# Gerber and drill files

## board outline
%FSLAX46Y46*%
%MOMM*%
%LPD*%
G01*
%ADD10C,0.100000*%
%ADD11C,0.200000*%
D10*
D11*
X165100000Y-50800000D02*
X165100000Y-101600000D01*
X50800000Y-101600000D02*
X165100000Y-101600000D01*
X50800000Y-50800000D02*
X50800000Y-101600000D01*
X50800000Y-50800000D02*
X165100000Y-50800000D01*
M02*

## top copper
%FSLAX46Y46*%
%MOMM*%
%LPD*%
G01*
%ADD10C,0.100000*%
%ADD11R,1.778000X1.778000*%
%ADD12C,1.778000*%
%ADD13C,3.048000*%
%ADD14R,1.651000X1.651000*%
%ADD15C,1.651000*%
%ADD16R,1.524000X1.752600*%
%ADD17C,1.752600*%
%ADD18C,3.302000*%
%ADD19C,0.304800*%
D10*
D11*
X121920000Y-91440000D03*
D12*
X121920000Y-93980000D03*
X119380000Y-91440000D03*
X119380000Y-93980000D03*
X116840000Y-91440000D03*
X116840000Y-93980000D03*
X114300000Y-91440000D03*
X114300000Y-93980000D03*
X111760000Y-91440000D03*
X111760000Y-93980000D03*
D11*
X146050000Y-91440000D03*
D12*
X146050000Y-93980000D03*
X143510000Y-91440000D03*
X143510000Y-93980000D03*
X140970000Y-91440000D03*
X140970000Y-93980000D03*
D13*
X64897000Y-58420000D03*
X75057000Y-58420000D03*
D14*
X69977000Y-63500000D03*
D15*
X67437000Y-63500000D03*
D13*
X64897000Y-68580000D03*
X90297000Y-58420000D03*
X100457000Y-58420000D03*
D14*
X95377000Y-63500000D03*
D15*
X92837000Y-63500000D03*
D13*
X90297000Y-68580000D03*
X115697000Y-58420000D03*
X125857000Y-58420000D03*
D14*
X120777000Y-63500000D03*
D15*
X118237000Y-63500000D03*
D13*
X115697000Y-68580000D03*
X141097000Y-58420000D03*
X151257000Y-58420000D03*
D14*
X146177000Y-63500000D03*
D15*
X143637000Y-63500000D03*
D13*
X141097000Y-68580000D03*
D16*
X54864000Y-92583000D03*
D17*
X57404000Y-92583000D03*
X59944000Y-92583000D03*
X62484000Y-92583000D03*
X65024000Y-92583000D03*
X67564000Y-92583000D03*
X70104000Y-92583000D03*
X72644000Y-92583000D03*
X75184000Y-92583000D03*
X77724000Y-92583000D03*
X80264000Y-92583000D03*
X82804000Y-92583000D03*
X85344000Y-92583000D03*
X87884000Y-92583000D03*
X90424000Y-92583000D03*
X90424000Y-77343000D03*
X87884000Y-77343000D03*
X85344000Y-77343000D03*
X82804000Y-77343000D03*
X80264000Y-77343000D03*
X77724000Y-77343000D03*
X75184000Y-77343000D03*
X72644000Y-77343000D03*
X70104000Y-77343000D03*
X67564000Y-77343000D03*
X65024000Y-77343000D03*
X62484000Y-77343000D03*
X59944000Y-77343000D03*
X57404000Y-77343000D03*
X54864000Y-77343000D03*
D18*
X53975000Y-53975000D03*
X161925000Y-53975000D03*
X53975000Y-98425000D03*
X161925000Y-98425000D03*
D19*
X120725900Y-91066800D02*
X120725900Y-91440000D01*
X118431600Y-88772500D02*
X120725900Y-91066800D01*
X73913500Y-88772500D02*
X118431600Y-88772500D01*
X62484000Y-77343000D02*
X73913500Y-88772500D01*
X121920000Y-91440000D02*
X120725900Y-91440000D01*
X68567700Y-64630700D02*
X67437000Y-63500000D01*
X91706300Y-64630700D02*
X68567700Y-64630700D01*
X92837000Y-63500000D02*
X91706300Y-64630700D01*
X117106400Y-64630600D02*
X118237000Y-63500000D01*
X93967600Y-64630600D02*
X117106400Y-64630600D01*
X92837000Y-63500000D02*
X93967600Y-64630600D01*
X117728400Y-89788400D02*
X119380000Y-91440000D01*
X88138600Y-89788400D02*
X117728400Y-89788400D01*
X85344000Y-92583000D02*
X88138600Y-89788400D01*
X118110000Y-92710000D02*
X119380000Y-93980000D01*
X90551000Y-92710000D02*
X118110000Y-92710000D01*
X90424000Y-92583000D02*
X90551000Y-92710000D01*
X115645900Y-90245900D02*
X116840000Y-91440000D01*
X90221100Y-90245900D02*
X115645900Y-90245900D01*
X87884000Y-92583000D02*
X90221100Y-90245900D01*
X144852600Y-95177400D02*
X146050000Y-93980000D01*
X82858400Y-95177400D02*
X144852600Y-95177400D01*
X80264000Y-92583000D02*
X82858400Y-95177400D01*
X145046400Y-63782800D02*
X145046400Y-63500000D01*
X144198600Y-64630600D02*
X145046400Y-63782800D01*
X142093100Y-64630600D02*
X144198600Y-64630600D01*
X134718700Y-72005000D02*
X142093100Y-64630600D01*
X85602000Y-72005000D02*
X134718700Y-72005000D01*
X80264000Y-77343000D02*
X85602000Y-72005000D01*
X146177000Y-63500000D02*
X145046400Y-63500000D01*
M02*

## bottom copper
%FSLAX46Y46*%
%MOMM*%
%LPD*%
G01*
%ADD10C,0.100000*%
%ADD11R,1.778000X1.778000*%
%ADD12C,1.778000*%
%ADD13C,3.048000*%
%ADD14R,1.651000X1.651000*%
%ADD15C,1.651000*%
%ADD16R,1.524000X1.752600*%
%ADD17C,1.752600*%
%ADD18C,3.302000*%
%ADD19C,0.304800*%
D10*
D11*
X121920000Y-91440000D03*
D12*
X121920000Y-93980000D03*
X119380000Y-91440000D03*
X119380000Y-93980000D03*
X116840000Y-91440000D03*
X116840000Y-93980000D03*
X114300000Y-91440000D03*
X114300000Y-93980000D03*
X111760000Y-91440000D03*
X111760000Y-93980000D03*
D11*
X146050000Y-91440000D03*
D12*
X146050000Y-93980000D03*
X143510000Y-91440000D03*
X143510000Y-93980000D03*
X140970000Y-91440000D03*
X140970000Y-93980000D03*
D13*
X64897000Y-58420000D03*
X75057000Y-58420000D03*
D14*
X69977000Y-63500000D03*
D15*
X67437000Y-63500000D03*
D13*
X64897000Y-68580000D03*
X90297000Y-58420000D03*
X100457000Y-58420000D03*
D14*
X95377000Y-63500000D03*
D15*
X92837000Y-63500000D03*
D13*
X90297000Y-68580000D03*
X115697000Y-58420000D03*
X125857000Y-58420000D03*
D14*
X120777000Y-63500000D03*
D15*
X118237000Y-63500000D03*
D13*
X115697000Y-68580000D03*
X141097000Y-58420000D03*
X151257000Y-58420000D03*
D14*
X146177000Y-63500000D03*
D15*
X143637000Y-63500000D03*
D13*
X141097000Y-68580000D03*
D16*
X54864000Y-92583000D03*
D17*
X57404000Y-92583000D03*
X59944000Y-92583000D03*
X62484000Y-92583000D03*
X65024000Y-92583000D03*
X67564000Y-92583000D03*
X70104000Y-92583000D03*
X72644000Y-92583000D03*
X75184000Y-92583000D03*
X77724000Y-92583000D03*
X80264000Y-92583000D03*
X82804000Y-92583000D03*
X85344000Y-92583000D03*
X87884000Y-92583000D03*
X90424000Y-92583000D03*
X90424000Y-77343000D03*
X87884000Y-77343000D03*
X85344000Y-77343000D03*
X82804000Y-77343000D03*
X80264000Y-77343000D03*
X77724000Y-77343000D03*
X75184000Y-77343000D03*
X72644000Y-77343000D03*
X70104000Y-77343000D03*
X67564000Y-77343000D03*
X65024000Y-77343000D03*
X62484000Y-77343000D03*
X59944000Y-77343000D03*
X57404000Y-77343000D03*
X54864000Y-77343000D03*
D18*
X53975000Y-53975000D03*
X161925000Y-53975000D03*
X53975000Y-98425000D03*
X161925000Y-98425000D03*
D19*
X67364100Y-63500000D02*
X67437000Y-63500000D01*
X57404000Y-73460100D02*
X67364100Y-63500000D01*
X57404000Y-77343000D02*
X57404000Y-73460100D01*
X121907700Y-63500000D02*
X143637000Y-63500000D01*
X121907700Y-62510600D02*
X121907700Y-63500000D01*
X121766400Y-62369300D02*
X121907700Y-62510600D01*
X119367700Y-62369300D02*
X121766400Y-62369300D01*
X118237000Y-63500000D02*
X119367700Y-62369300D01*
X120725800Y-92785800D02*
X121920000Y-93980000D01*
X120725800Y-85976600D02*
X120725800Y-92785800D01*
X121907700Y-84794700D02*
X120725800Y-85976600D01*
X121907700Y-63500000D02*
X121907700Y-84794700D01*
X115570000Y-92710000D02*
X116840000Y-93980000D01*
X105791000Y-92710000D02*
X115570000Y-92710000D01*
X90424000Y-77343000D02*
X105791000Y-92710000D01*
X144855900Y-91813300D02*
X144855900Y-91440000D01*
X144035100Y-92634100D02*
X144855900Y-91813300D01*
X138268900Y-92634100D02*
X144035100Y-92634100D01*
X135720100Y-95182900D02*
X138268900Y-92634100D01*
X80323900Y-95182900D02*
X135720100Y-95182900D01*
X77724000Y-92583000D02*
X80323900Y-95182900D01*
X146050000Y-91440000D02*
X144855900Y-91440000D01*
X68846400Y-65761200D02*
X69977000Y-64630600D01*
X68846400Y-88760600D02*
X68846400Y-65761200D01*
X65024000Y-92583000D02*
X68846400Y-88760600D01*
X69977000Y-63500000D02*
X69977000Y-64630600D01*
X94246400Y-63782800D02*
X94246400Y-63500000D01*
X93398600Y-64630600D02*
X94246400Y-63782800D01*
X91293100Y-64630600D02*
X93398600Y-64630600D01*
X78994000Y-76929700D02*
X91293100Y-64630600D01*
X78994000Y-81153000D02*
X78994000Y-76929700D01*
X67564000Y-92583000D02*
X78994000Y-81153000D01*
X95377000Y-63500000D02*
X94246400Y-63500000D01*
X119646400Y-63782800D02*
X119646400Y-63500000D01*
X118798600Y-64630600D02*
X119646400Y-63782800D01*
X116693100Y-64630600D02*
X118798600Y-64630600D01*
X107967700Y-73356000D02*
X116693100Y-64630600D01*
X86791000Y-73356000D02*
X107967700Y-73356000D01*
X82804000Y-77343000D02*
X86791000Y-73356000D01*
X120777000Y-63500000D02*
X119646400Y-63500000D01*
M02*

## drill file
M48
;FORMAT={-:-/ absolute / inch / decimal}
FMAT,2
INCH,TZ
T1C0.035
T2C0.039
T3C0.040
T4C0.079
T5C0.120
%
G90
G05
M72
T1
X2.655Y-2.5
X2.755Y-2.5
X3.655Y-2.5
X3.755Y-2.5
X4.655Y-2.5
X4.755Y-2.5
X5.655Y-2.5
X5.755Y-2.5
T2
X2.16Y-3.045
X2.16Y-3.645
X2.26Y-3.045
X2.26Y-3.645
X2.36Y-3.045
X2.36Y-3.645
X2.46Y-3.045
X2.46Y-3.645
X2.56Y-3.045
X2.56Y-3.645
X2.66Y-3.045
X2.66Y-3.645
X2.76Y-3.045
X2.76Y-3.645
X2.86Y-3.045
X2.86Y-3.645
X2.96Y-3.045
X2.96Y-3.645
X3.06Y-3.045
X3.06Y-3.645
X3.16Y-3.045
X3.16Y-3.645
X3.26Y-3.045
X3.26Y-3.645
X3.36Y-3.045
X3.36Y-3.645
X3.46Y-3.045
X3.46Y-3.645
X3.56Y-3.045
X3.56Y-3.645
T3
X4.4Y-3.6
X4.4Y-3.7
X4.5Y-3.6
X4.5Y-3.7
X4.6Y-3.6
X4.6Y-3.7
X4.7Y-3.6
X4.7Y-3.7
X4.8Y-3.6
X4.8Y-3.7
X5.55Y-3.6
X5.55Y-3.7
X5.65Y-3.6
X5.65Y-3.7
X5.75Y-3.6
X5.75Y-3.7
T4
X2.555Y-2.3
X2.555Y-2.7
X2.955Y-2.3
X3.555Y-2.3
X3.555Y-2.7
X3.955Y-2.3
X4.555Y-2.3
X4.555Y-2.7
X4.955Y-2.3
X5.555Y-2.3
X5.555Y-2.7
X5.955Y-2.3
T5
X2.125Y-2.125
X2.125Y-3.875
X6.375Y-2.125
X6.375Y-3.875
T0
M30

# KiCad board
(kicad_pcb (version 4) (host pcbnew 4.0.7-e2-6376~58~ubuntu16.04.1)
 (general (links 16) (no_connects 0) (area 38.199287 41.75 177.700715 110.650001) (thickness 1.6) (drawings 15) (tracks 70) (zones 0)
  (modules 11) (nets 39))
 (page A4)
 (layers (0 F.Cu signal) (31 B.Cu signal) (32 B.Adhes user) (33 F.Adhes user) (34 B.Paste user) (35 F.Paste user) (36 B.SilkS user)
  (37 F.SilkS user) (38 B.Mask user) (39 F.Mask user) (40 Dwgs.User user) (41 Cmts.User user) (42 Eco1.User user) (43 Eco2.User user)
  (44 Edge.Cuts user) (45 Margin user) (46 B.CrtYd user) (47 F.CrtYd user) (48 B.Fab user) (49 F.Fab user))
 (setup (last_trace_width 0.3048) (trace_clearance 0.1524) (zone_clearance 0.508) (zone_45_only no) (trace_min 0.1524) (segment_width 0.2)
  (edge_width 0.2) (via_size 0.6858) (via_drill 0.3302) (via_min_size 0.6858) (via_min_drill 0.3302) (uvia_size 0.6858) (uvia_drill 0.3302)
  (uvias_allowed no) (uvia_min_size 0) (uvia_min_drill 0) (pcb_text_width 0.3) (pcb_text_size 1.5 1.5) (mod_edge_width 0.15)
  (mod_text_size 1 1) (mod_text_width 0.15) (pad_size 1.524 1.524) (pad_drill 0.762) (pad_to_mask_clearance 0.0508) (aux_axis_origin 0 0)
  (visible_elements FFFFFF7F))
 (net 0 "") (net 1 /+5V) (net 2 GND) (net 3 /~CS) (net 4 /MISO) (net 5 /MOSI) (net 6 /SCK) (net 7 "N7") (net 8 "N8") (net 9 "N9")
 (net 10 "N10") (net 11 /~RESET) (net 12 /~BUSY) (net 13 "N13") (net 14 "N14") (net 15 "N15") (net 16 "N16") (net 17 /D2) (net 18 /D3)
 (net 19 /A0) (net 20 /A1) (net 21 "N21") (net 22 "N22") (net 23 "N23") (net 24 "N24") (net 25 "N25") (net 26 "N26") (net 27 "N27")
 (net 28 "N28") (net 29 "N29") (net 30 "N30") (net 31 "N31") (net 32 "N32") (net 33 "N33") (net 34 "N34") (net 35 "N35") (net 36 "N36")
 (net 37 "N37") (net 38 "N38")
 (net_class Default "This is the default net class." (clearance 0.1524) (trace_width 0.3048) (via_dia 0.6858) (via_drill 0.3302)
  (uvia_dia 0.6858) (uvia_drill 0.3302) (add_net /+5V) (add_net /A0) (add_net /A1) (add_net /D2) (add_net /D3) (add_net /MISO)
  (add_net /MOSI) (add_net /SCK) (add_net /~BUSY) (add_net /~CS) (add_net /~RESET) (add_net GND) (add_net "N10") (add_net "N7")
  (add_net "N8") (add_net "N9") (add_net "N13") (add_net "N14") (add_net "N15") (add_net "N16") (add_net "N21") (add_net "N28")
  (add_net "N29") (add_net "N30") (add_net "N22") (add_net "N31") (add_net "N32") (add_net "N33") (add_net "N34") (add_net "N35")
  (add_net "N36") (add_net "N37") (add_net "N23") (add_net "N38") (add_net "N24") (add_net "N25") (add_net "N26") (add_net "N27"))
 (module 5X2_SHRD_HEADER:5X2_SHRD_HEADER (layer F.Cu) (at 116.84 92.71 180)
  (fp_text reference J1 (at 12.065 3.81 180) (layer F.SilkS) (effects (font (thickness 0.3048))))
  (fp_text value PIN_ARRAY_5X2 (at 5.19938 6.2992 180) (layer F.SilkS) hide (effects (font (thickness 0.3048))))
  (pad 1 thru_hole rect (at -5.08 1.27 180) (size 1.778 1.778) (drill 1.016) (layers *.Cu *.Mask F.SilkS) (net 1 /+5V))
  (pad 2 thru_hole circle (at -5.08 -1.27 180) (size 1.778 1.778) (drill 1.016) (layers *.Cu *.Mask F.SilkS) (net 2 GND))
  (pad 3 thru_hole circle (at -2.54 1.27 180) (size 1.778 1.778) (drill 1.016) (layers *.Cu *.Mask F.SilkS) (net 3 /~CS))
  (pad 4 thru_hole circle (at -2.54 -1.27 180) (size 1.778 1.778) (drill 1.016) (layers *.Cu *.Mask F.SilkS) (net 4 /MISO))
  (pad 5 thru_hole circle (at 0 1.27 180) (size 1.778 1.778) (drill 1.016) (layers *.Cu *.Mask F.SilkS) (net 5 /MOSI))
  (pad 6 thru_hole circle (at 0 -1.27 180) (size 1.778 1.778) (drill 1.016) (layers *.Cu *.Mask F.SilkS) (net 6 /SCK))
  (pad 7 thru_hole circle (at 2.54 1.27 180) (size 1.778 1.778) (drill 1.016) (layers *.Cu *.Mask F.SilkS) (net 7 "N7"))
  (pad 8 thru_hole circle (at 2.54 -1.27 180) (size 1.778 1.778) (drill 1.016) (layers *.Cu *.Mask F.SilkS) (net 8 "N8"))
  (pad 9 thru_hole circle (at 5.08 1.27 180) (size 1.778 1.778) (drill 1.016) (layers *.Cu *.Mask F.SilkS) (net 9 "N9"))
  (pad 10 thru_hole circle (at 5.08 -1.27 180) (size 1.778 1.778) (drill 1.016) (layers *.Cu *.Mask F.SilkS) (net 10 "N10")))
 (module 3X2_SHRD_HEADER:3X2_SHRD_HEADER (layer F.Cu) (at 143.51 92.71 180)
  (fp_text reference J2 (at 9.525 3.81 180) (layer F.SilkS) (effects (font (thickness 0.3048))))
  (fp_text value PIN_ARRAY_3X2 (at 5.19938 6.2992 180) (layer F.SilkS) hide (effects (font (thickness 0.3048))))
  (pad 1 thru_hole rect (at -2.54 1.27 180) (size 1.778 1.778) (drill 1.016) (layers *.Cu *.Mask F.SilkS) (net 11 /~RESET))
  (pad 2 thru_hole circle (at -2.54 -1.27 180) (size 1.778 1.778) (drill 1.016) (layers *.Cu *.Mask F.SilkS) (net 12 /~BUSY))
  (pad 3 thru_hole circle (at 0 1.27 180) (size 1.778 1.778) (drill 1.016) (layers *.Cu *.Mask F.SilkS) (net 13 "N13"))
  (pad 4 thru_hole circle (at 0 -1.27 180) (size 1.778 1.778) (drill 1.016) (layers *.Cu *.Mask F.SilkS) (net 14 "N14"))
  (pad 5 thru_hole circle (at 2.54 1.27 180) (size 1.778 1.778) (drill 1.016) (layers *.Cu *.Mask F.SilkS) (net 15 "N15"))
  (pad 6 thru_hole circle (at 2.54 -1.27 180) (size 1.778 1.778) (drill 1.016) (layers *.Cu *.Mask F.SilkS) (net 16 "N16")))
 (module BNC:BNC (layer F.Cu) (at 69.977 58.42)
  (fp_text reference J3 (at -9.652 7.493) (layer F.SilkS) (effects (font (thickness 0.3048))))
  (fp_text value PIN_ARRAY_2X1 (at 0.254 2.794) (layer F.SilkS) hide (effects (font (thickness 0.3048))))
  (pad "" thru_hole circle (at -5.08 0) (size 3.048 3.048) (drill 2.00914) (layers *.Cu *.Mask))
  (pad "" thru_hole circle (at 5.08 0) (size 3.048 3.048) (drill 2.00914) (layers *.Cu *.Mask))
  (pad 1 thru_hole rect (at 0 5.08) (size 1.651 1.651) (drill 0.889) (layers *.Cu *.Mask) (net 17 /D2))
  (pad 2 thru_hole circle (at -2.54 5.08) (size 1.651 1.651) (drill 0.889) (layers *.Cu *.Mask) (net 2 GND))
  (pad "" thru_hole circle (at -5.08 10.16) (size 3.048 3.048) (drill 2.00914) (layers *.Cu *.Mask)))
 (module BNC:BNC (layer F.Cu) (at 95.377 58.42)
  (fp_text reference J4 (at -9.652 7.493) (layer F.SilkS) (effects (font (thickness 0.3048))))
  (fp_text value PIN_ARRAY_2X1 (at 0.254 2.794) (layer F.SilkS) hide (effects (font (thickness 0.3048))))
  (pad "" thru_hole circle (at -5.08 0) (size 3.048 3.048) (drill 2.00914) (layers *.Cu *.Mask))
  (pad "" thru_hole circle (at 5.08 0) (size 3.048 3.048) (drill 2.00914) (layers *.Cu *.Mask))
  (pad 1 thru_hole rect (at 0 5.08) (size 1.651 1.651) (drill 0.889) (layers *.Cu *.Mask) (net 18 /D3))
  (pad 2 thru_hole circle (at -2.54 5.08) (size 1.651 1.651) (drill 0.889) (layers *.Cu *.Mask) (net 2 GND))
  (pad "" thru_hole circle (at -5.08 10.16) (size 3.048 3.048) (drill 2.00914) (layers *.Cu *.Mask)))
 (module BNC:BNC (layer F.Cu) (at 120.777 58.42)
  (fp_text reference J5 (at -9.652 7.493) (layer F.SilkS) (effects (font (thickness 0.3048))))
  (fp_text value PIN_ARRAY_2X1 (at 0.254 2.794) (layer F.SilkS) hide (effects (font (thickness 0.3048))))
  (pad "" thru_hole circle (at -5.08 0) (size 3.048 3.048) (drill 2.00914) (layers *.Cu *.Mask))
  (pad "" thru_hole circle (at 5.08 0) (size 3.048 3.048) (drill 2.00914) (layers *.Cu *.Mask))
  (pad 1 thru_hole rect (at 0 5.08) (size 1.651 1.651) (drill 0.889) (layers *.Cu *.Mask) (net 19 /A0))
  (pad 2 thru_hole circle (at -2.54 5.08) (size 1.651 1.651) (drill 0.889) (layers *.Cu *.Mask) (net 2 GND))
  (pad "" thru_hole circle (at -5.08 10.16) (size 3.048 3.048) (drill 2.00914) (layers *.Cu *.Mask)))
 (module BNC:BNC (layer F.Cu) (at 146.177 58.42)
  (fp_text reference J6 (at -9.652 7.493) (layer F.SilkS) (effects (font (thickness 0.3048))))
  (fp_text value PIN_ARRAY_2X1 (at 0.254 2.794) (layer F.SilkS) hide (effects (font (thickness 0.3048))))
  (pad "" thru_hole circle (at -5.08 0) (size 3.048 3.048) (drill 2.00914) (layers *.Cu *.Mask))
  (pad "" thru_hole circle (at 5.08 0) (size 3.048 3.048) (drill 2.00914) (layers *.Cu *.Mask))
  (pad 1 thru_hole rect (at 0 5.08) (size 1.651 1.651) (drill 0.889) (layers *.Cu *.Mask) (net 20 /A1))
  (pad 2 thru_hole circle (at -2.54 5.08) (size 1.651 1.651) (drill 0.889) (layers *.Cu *.Mask) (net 2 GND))
  (pad "" thru_hole circle (at -5.08 10.16) (size 3.048 3.048) (drill 2.00914) (layers *.Cu *.Mask)))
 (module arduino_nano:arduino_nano (layer F.Cu) (at 72.644 84.963 90)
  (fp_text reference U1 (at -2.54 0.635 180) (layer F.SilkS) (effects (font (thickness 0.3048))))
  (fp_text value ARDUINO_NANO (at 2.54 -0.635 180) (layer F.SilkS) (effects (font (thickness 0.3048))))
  (pad 1 thru_hole rect (at -7.62 -17.78 90) (size 1.7526 1.524) (drill 0.9906) (layers *.Cu *.Mask F.SilkS) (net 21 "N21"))
  (pad 2 thru_hole circle (at -7.62 -15.24 90) (size 1.7526 1.7526) (drill 0.9906) (layers *.Cu *.Mask F.SilkS) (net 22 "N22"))
  (pad 3 thru_hole circle (at -7.62 -12.7 90) (size 1.7526 1.7526) (drill 0.9906) (layers *.Cu *.Mask F.SilkS) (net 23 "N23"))
  (pad 4 thru_hole circle (at -7.62 -10.16 90) (size 1.7526 1.7526) (drill 0.9906) (layers *.Cu *.Mask F.SilkS) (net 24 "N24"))
  (pad 5 thru_hole circle (at -7.62 -7.62 90) (size 1.7526 1.7526) (drill 0.9906) (layers *.Cu *.Mask F.SilkS) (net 17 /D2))
  (pad 6 thru_hole circle (at -7.62 -5.08 90) (size 1.7526 1.7526) (drill 0.9906) (layers *.Cu *.Mask F.SilkS) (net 18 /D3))
  (pad 7 thru_hole circle (at -7.62 -2.54 90) (size 1.7526 1.7526) (drill 0.9906) (layers *.Cu *.Mask F.SilkS) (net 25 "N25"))
  (pad 8 thru_hole circle (at -7.62 0 90) (size 1.7526 1.7526) (drill 0.9906) (layers *.Cu *.Mask F.SilkS) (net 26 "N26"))
  (pad 9 thru_hole circle (at -7.62 2.54 90) (size 1.7526 1.7526) (drill 0.9906) (layers *.Cu *.Mask F.SilkS) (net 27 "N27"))
  (pad 10 thru_hole circle (at -7.62 5.08 90) (size 1.7526 1.7526) (drill 0.9906) (layers *.Cu *.Mask F.SilkS) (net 11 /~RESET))
  (pad 11 thru_hole circle (at -7.62 7.62 90) (size 1.7526 1.7526) (drill 0.9906) (layers *.Cu *.Mask F.SilkS) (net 12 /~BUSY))
  (pad 12 thru_hole circle (at -7.62 10.16 90) (size 1.7526 1.7526) (drill 0.9906) (layers *.Cu *.Mask F.SilkS) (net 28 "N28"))
  (pad 13 thru_hole circle (at -7.62 12.7 90) (size 1.7526 1.7526) (drill 0.9906) (layers *.Cu *.Mask F.SilkS) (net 3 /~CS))
  (pad 14 thru_hole circle (at -7.62 15.24 90) (size 1.7526 1.7526) (drill 0.9906) (layers *.Cu *.Mask F.SilkS) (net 5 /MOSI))
  (pad 15 thru_hole circle (at -7.62 17.78 90) (size 1.7526 1.7526) (drill 0.9906) (layers *.Cu *.Mask F.SilkS) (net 4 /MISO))
  (pad 16 thru_hole circle (at 7.62 17.78 90) (size 1.7526 1.7526) (drill 0.9906) (layers *.Cu *.Mask F.SilkS) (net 6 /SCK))
  (pad 17 thru_hole circle (at 7.62 15.24 90) (size 1.7526 1.7526) (drill 0.9906) (layers *.Cu *.Mask F.SilkS) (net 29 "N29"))
  (pad 18 thru_hole circle (at 7.62 12.7 90) (size 1.7526 1.7526) (drill 0.9906) (layers *.Cu *.Mask F.SilkS) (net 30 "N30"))
  (pad 19 thru_hole circle (at 7.62 10.16 90) (size 1.7526 1.7526) (drill 0.9906) (layers *.Cu *.Mask F.SilkS) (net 19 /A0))
  (pad 20 thru_hole circle (at 7.62 7.62 90) (size 1.7526 1.7526) (drill 0.9906) (layers *.Cu *.Mask F.SilkS) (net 20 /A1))
  (pad 21 thru_hole circle (at 7.62 5.08 90) (size 1.7526 1.7526) (drill 0.9906) (layers *.Cu *.Mask F.SilkS) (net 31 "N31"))
  (pad 22 thru_hole circle (at 7.62 2.54 90) (size 1.7526 1.7526) (drill 0.9906) (layers *.Cu *.Mask F.SilkS) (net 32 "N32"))
  (pad 23 thru_hole circle (at 7.62 0 90) (size 1.7526 1.7526) (drill 0.9906) (layers *.Cu *.Mask F.SilkS) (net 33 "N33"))
  (pad 24 thru_hole circle (at 7.62 -2.54 90) (size 1.7526 1.7526) (drill 0.9906) (layers *.Cu *.Mask F.SilkS) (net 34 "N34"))
  (pad 25 thru_hole circle (at 7.62 -5.08 90) (size 1.7526 1.7526) (drill 0.9906) (layers *.Cu *.Mask F.SilkS) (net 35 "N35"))
  (pad 26 thru_hole circle (at 7.62 -7.62 90) (size 1.7526 1.7526) (drill 0.9906) (layers *.Cu *.Mask F.SilkS) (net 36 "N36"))
  (pad 27 thru_hole circle (at 7.62 -10.16 90) (size 1.7526 1.7526) (drill 0.9906) (layers *.Cu *.Mask F.SilkS) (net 1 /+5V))
  (pad 28 thru_hole circle (at 7.62 -12.7 90) (size 1.7526 1.7526) (drill 0.9906) (layers *.Cu *.Mask F.SilkS) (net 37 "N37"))
  (pad 29 thru_hole circle (at 7.62 -15.24 90) (size 1.7526 1.7526) (drill 0.9906) (layers *.Cu *.Mask F.SilkS) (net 2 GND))
  (pad 30 thru_hole circle (at 7.62 -17.78 90) (size 1.7526 1.7526) (drill 0.9906) (layers *.Cu *.Mask F.SilkS) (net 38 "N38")))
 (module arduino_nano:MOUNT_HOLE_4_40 (layer F.Cu) (at 53.975 53.975)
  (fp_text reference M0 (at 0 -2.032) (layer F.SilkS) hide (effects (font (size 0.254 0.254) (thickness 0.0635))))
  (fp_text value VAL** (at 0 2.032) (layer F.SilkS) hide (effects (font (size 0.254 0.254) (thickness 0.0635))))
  (pad "" thru_hole circle (at 0 0) (size 3.302 3.302) (drill 3.048) (layers *.Cu *.SilkS *.Mask)))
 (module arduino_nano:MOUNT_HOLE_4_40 (layer F.Cu) (at 161.925 53.975)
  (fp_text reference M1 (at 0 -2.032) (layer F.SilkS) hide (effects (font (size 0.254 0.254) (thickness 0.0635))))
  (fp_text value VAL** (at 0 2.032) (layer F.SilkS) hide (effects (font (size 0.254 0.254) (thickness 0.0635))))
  (pad "" thru_hole circle (at 0 0) (size 3.302 3.302) (drill 3.048) (layers *.Cu *.SilkS *.Mask)))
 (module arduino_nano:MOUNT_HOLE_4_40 (layer F.Cu) (at 53.975 98.425)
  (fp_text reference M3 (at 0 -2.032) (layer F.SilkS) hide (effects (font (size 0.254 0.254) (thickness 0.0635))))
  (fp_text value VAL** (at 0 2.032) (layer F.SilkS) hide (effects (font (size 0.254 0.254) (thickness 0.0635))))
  (pad "" thru_hole circle (at 0 0) (size 3.302 3.302) (drill 3.048) (layers *.Cu *.SilkS *.Mask)))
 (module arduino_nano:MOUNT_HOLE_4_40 (layer F.Cu) (at 161.925 98.425)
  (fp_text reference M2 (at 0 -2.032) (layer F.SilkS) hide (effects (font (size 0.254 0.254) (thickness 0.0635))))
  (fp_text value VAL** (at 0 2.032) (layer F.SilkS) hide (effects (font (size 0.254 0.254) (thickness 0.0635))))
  (pad "" thru_hole circle (at 0 0) (size 3.302 3.302) (drill 3.048) (layers *.Cu *.SilkS *.Mask)))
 (gr_line (start 165.1 50.8) (end 165.1 101.6) (angle 90) (layer Edge.Cuts) (width 0.2))
 (gr_line (start 50.8 101.6) (end 165.1 101.6) (angle 90) (layer Edge.Cuts) (width 0.2))
 (gr_line (start 50.8 50.8) (end 50.8 101.6) (angle 90) (layer Edge.Cuts) (width 0.2))
 (gr_line (start 50.8 50.8) (end 165.1 50.8) (angle 90) (layer Edge.Cuts) (width 0.2))
 (segment (start 120.7259 91.0668) (end 120.7259 91.44) (width 0.3048) (layer F.Cu) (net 1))
 (segment (start 118.4316 88.7725) (end 120.7259 91.0668) (width 0.3048) (layer F.Cu) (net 1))
 (segment (start 73.9135 88.7725) (end 118.4316 88.7725) (width 0.3048) (layer F.Cu) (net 1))
 (segment (start 62.484 77.343) (end 73.9135 88.7725) (width 0.3048) (layer F.Cu) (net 1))
 (segment (start 121.92 91.44) (end 120.7259 91.44) (width 0.3048) (layer F.Cu) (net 1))
 (segment (start 67.3641 63.5) (end 67.437 63.5) (width 0.3048) (layer B.Cu) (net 2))
 (segment (start 57.404 73.4601) (end 67.3641 63.5) (width 0.3048) (layer B.Cu) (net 2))
 (segment (start 57.404 77.343) (end 57.404 73.4601) (width 0.3048) (layer B.Cu) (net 2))
 (segment (start 68.5677 64.6307) (end 67.437 63.5) (width 0.3048) (layer F.Cu) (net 2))
 (segment (start 91.7063 64.6307) (end 68.5677 64.6307) (width 0.3048) (layer F.Cu) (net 2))
 (segment (start 92.837 63.5) (end 91.7063 64.6307) (width 0.3048) (layer F.Cu) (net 2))
 (segment (start 117.1064 64.6306) (end 118.237 63.5) (width 0.3048) (layer F.Cu) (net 2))
 (segment (start 93.9676 64.6306) (end 117.1064 64.6306) (width 0.3048) (layer F.Cu) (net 2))
 (segment (start 92.837 63.5) (end 93.9676 64.6306) (width 0.3048) (layer F.Cu) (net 2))
 (segment (start 121.9077 63.5) (end 143.637 63.5) (width 0.3048) (layer B.Cu) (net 2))
 (segment (start 121.9077 62.5106) (end 121.9077 63.5) (width 0.3048) (layer B.Cu) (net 2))
 (segment (start 121.7664 62.3693) (end 121.9077 62.5106) (width 0.3048) (layer B.Cu) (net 2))
 (segment (start 119.3677 62.3693) (end 121.7664 62.3693) (width 0.3048) (layer B.Cu) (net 2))
 (segment (start 118.237 63.5) (end 119.3677 62.3693) (width 0.3048) (layer B.Cu) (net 2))
 (segment (start 120.7258 92.7858) (end 121.92 93.98) (width 0.3048) (layer B.Cu) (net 2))
 (segment (start 120.7258 85.9766) (end 120.7258 92.7858) (width 0.3048) (layer B.Cu) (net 2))
 (segment (start 121.9077 84.7947) (end 120.7258 85.9766) (width 0.3048) (layer B.Cu) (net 2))
 (segment (start 121.9077 63.5) (end 121.9077 84.7947) (width 0.3048) (layer B.Cu) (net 2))
 (segment (start 117.7284 89.7884) (end 119.38 91.44) (width 0.3048) (layer F.Cu) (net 3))
 (segment (start 88.1386 89.7884) (end 117.7284 89.7884) (width 0.3048) (layer F.Cu) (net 3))
 (segment (start 85.344 92.583) (end 88.1386 89.7884) (width 0.3048) (layer F.Cu) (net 3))
 (segment (start 118.11 92.71) (end 119.38 93.98) (width 0.3048) (layer F.Cu) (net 4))
 (segment (start 90.551 92.71) (end 118.11 92.71) (width 0.3048) (layer F.Cu) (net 4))
 (segment (start 90.424 92.583) (end 90.551 92.71) (width 0.3048) (layer F.Cu) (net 4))
 (segment (start 115.6459 90.2459) (end 116.84 91.44) (width 0.3048) (layer F.Cu) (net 5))
 (segment (start 90.2211 90.2459) (end 115.6459 90.2459) (width 0.3048) (layer F.Cu) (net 5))
 (segment (start 87.884 92.583) (end 90.2211 90.2459) (width 0.3048) (layer F.Cu) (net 5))
 (segment (start 115.57 92.71) (end 116.84 93.98) (width 0.3048) (layer B.Cu) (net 6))
 (segment (start 105.791 92.71) (end 115.57 92.71) (width 0.3048) (layer B.Cu) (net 6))
 (segment (start 90.424 77.343) (end 105.791 92.71) (width 0.3048) (layer B.Cu) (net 6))
 (segment (start 144.8559 91.8133) (end 144.8559 91.44) (width 0.3048) (layer B.Cu) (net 11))
 (segment (start 144.0351 92.6341) (end 144.8559 91.8133) (width 0.3048) (layer B.Cu) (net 11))
 (segment (start 138.2689 92.6341) (end 144.0351 92.6341) (width 0.3048) (layer B.Cu) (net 11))
 (segment (start 135.7201 95.1829) (end 138.2689 92.6341) (width 0.3048) (layer B.Cu) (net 11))
 (segment (start 80.3239 95.1829) (end 135.7201 95.1829) (width 0.3048) (layer B.Cu) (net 11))
 (segment (start 77.724 92.583) (end 80.3239 95.1829) (width 0.3048) (layer B.Cu) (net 11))
 (segment (start 146.05 91.44) (end 144.8559 91.44) (width 0.3048) (layer B.Cu) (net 11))
 (segment (start 144.8526 95.1774) (end 146.05 93.98) (width 0.3048) (layer F.Cu) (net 12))
 (segment (start 82.8584 95.1774) (end 144.8526 95.1774) (width 0.3048) (layer F.Cu) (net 12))
 (segment (start 80.264 92.583) (end 82.8584 95.1774) (width 0.3048) (layer F.Cu) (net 12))
 (segment (start 68.8464 65.7612) (end 69.977 64.6306) (width 0.3048) (layer B.Cu) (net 17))
 (segment (start 68.8464 88.7606) (end 68.8464 65.7612) (width 0.3048) (layer B.Cu) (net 17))
 (segment (start 65.024 92.583) (end 68.8464 88.7606) (width 0.3048) (layer B.Cu) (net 17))
 (segment (start 69.977 63.5) (end 69.977 64.6306) (width 0.3048) (layer B.Cu) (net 17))
 (segment (start 94.2464 63.7828) (end 94.2464 63.5) (width 0.3048) (layer B.Cu) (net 18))
 (segment (start 93.3986 64.6306) (end 94.2464 63.7828) (width 0.3048) (layer B.Cu) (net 18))
 (segment (start 91.2931 64.6306) (end 93.3986 64.6306) (width 0.3048) (layer B.Cu) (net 18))
 (segment (start 78.994 76.9297) (end 91.2931 64.6306) (width 0.3048) (layer B.Cu) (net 18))
 (segment (start 78.994 81.153) (end 78.994 76.9297) (width 0.3048) (layer B.Cu) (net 18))
 (segment (start 67.564 92.583) (end 78.994 81.153) (width 0.3048) (layer B.Cu) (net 18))
 (segment (start 95.377 63.5) (end 94.2464 63.5) (width 0.3048) (layer B.Cu) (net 18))
 (segment (start 119.6464 63.7828) (end 119.6464 63.5) (width 0.3048) (layer B.Cu) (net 19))
 (segment (start 118.7986 64.6306) (end 119.6464 63.7828) (width 0.3048) (layer B.Cu) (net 19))
 (segment (start 116.6931 64.6306) (end 118.7986 64.6306) (width 0.3048) (layer B.Cu) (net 19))
 (segment (start 107.9677 73.356) (end 116.6931 64.6306) (width 0.3048) (layer B.Cu) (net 19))
 (segment (start 86.791 73.356) (end 107.9677 73.356) (width 0.3048) (layer B.Cu) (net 19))
 (segment (start 82.804 77.343) (end 86.791 73.356) (width 0.3048) (layer B.Cu) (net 19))
 (segment (start 120.777 63.5) (end 119.6464 63.5) (width 0.3048) (layer B.Cu) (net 19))
 (segment (start 145.0464 63.7828) (end 145.0464 63.5) (width 0.3048) (layer F.Cu) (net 20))
 (segment (start 144.1986 64.6306) (end 145.0464 63.7828) (width 0.3048) (layer F.Cu) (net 20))
 (segment (start 142.0931 64.6306) (end 144.1986 64.6306) (width 0.3048) (layer F.Cu) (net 20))
 (segment (start 134.7187 72.005) (end 142.0931 64.6306) (width 0.3048) (layer F.Cu) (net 20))
 (segment (start 85.602 72.005) (end 134.7187 72.005) (width 0.3048) (layer F.Cu) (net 20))
 (segment (start 80.264 77.343) (end 85.602 72.005) (width 0.3048) (layer F.Cu) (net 20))
 (segment (start 146.177 63.5) (end 145.0464 63.5) (width 0.3048) (layer F.Cu) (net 20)))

